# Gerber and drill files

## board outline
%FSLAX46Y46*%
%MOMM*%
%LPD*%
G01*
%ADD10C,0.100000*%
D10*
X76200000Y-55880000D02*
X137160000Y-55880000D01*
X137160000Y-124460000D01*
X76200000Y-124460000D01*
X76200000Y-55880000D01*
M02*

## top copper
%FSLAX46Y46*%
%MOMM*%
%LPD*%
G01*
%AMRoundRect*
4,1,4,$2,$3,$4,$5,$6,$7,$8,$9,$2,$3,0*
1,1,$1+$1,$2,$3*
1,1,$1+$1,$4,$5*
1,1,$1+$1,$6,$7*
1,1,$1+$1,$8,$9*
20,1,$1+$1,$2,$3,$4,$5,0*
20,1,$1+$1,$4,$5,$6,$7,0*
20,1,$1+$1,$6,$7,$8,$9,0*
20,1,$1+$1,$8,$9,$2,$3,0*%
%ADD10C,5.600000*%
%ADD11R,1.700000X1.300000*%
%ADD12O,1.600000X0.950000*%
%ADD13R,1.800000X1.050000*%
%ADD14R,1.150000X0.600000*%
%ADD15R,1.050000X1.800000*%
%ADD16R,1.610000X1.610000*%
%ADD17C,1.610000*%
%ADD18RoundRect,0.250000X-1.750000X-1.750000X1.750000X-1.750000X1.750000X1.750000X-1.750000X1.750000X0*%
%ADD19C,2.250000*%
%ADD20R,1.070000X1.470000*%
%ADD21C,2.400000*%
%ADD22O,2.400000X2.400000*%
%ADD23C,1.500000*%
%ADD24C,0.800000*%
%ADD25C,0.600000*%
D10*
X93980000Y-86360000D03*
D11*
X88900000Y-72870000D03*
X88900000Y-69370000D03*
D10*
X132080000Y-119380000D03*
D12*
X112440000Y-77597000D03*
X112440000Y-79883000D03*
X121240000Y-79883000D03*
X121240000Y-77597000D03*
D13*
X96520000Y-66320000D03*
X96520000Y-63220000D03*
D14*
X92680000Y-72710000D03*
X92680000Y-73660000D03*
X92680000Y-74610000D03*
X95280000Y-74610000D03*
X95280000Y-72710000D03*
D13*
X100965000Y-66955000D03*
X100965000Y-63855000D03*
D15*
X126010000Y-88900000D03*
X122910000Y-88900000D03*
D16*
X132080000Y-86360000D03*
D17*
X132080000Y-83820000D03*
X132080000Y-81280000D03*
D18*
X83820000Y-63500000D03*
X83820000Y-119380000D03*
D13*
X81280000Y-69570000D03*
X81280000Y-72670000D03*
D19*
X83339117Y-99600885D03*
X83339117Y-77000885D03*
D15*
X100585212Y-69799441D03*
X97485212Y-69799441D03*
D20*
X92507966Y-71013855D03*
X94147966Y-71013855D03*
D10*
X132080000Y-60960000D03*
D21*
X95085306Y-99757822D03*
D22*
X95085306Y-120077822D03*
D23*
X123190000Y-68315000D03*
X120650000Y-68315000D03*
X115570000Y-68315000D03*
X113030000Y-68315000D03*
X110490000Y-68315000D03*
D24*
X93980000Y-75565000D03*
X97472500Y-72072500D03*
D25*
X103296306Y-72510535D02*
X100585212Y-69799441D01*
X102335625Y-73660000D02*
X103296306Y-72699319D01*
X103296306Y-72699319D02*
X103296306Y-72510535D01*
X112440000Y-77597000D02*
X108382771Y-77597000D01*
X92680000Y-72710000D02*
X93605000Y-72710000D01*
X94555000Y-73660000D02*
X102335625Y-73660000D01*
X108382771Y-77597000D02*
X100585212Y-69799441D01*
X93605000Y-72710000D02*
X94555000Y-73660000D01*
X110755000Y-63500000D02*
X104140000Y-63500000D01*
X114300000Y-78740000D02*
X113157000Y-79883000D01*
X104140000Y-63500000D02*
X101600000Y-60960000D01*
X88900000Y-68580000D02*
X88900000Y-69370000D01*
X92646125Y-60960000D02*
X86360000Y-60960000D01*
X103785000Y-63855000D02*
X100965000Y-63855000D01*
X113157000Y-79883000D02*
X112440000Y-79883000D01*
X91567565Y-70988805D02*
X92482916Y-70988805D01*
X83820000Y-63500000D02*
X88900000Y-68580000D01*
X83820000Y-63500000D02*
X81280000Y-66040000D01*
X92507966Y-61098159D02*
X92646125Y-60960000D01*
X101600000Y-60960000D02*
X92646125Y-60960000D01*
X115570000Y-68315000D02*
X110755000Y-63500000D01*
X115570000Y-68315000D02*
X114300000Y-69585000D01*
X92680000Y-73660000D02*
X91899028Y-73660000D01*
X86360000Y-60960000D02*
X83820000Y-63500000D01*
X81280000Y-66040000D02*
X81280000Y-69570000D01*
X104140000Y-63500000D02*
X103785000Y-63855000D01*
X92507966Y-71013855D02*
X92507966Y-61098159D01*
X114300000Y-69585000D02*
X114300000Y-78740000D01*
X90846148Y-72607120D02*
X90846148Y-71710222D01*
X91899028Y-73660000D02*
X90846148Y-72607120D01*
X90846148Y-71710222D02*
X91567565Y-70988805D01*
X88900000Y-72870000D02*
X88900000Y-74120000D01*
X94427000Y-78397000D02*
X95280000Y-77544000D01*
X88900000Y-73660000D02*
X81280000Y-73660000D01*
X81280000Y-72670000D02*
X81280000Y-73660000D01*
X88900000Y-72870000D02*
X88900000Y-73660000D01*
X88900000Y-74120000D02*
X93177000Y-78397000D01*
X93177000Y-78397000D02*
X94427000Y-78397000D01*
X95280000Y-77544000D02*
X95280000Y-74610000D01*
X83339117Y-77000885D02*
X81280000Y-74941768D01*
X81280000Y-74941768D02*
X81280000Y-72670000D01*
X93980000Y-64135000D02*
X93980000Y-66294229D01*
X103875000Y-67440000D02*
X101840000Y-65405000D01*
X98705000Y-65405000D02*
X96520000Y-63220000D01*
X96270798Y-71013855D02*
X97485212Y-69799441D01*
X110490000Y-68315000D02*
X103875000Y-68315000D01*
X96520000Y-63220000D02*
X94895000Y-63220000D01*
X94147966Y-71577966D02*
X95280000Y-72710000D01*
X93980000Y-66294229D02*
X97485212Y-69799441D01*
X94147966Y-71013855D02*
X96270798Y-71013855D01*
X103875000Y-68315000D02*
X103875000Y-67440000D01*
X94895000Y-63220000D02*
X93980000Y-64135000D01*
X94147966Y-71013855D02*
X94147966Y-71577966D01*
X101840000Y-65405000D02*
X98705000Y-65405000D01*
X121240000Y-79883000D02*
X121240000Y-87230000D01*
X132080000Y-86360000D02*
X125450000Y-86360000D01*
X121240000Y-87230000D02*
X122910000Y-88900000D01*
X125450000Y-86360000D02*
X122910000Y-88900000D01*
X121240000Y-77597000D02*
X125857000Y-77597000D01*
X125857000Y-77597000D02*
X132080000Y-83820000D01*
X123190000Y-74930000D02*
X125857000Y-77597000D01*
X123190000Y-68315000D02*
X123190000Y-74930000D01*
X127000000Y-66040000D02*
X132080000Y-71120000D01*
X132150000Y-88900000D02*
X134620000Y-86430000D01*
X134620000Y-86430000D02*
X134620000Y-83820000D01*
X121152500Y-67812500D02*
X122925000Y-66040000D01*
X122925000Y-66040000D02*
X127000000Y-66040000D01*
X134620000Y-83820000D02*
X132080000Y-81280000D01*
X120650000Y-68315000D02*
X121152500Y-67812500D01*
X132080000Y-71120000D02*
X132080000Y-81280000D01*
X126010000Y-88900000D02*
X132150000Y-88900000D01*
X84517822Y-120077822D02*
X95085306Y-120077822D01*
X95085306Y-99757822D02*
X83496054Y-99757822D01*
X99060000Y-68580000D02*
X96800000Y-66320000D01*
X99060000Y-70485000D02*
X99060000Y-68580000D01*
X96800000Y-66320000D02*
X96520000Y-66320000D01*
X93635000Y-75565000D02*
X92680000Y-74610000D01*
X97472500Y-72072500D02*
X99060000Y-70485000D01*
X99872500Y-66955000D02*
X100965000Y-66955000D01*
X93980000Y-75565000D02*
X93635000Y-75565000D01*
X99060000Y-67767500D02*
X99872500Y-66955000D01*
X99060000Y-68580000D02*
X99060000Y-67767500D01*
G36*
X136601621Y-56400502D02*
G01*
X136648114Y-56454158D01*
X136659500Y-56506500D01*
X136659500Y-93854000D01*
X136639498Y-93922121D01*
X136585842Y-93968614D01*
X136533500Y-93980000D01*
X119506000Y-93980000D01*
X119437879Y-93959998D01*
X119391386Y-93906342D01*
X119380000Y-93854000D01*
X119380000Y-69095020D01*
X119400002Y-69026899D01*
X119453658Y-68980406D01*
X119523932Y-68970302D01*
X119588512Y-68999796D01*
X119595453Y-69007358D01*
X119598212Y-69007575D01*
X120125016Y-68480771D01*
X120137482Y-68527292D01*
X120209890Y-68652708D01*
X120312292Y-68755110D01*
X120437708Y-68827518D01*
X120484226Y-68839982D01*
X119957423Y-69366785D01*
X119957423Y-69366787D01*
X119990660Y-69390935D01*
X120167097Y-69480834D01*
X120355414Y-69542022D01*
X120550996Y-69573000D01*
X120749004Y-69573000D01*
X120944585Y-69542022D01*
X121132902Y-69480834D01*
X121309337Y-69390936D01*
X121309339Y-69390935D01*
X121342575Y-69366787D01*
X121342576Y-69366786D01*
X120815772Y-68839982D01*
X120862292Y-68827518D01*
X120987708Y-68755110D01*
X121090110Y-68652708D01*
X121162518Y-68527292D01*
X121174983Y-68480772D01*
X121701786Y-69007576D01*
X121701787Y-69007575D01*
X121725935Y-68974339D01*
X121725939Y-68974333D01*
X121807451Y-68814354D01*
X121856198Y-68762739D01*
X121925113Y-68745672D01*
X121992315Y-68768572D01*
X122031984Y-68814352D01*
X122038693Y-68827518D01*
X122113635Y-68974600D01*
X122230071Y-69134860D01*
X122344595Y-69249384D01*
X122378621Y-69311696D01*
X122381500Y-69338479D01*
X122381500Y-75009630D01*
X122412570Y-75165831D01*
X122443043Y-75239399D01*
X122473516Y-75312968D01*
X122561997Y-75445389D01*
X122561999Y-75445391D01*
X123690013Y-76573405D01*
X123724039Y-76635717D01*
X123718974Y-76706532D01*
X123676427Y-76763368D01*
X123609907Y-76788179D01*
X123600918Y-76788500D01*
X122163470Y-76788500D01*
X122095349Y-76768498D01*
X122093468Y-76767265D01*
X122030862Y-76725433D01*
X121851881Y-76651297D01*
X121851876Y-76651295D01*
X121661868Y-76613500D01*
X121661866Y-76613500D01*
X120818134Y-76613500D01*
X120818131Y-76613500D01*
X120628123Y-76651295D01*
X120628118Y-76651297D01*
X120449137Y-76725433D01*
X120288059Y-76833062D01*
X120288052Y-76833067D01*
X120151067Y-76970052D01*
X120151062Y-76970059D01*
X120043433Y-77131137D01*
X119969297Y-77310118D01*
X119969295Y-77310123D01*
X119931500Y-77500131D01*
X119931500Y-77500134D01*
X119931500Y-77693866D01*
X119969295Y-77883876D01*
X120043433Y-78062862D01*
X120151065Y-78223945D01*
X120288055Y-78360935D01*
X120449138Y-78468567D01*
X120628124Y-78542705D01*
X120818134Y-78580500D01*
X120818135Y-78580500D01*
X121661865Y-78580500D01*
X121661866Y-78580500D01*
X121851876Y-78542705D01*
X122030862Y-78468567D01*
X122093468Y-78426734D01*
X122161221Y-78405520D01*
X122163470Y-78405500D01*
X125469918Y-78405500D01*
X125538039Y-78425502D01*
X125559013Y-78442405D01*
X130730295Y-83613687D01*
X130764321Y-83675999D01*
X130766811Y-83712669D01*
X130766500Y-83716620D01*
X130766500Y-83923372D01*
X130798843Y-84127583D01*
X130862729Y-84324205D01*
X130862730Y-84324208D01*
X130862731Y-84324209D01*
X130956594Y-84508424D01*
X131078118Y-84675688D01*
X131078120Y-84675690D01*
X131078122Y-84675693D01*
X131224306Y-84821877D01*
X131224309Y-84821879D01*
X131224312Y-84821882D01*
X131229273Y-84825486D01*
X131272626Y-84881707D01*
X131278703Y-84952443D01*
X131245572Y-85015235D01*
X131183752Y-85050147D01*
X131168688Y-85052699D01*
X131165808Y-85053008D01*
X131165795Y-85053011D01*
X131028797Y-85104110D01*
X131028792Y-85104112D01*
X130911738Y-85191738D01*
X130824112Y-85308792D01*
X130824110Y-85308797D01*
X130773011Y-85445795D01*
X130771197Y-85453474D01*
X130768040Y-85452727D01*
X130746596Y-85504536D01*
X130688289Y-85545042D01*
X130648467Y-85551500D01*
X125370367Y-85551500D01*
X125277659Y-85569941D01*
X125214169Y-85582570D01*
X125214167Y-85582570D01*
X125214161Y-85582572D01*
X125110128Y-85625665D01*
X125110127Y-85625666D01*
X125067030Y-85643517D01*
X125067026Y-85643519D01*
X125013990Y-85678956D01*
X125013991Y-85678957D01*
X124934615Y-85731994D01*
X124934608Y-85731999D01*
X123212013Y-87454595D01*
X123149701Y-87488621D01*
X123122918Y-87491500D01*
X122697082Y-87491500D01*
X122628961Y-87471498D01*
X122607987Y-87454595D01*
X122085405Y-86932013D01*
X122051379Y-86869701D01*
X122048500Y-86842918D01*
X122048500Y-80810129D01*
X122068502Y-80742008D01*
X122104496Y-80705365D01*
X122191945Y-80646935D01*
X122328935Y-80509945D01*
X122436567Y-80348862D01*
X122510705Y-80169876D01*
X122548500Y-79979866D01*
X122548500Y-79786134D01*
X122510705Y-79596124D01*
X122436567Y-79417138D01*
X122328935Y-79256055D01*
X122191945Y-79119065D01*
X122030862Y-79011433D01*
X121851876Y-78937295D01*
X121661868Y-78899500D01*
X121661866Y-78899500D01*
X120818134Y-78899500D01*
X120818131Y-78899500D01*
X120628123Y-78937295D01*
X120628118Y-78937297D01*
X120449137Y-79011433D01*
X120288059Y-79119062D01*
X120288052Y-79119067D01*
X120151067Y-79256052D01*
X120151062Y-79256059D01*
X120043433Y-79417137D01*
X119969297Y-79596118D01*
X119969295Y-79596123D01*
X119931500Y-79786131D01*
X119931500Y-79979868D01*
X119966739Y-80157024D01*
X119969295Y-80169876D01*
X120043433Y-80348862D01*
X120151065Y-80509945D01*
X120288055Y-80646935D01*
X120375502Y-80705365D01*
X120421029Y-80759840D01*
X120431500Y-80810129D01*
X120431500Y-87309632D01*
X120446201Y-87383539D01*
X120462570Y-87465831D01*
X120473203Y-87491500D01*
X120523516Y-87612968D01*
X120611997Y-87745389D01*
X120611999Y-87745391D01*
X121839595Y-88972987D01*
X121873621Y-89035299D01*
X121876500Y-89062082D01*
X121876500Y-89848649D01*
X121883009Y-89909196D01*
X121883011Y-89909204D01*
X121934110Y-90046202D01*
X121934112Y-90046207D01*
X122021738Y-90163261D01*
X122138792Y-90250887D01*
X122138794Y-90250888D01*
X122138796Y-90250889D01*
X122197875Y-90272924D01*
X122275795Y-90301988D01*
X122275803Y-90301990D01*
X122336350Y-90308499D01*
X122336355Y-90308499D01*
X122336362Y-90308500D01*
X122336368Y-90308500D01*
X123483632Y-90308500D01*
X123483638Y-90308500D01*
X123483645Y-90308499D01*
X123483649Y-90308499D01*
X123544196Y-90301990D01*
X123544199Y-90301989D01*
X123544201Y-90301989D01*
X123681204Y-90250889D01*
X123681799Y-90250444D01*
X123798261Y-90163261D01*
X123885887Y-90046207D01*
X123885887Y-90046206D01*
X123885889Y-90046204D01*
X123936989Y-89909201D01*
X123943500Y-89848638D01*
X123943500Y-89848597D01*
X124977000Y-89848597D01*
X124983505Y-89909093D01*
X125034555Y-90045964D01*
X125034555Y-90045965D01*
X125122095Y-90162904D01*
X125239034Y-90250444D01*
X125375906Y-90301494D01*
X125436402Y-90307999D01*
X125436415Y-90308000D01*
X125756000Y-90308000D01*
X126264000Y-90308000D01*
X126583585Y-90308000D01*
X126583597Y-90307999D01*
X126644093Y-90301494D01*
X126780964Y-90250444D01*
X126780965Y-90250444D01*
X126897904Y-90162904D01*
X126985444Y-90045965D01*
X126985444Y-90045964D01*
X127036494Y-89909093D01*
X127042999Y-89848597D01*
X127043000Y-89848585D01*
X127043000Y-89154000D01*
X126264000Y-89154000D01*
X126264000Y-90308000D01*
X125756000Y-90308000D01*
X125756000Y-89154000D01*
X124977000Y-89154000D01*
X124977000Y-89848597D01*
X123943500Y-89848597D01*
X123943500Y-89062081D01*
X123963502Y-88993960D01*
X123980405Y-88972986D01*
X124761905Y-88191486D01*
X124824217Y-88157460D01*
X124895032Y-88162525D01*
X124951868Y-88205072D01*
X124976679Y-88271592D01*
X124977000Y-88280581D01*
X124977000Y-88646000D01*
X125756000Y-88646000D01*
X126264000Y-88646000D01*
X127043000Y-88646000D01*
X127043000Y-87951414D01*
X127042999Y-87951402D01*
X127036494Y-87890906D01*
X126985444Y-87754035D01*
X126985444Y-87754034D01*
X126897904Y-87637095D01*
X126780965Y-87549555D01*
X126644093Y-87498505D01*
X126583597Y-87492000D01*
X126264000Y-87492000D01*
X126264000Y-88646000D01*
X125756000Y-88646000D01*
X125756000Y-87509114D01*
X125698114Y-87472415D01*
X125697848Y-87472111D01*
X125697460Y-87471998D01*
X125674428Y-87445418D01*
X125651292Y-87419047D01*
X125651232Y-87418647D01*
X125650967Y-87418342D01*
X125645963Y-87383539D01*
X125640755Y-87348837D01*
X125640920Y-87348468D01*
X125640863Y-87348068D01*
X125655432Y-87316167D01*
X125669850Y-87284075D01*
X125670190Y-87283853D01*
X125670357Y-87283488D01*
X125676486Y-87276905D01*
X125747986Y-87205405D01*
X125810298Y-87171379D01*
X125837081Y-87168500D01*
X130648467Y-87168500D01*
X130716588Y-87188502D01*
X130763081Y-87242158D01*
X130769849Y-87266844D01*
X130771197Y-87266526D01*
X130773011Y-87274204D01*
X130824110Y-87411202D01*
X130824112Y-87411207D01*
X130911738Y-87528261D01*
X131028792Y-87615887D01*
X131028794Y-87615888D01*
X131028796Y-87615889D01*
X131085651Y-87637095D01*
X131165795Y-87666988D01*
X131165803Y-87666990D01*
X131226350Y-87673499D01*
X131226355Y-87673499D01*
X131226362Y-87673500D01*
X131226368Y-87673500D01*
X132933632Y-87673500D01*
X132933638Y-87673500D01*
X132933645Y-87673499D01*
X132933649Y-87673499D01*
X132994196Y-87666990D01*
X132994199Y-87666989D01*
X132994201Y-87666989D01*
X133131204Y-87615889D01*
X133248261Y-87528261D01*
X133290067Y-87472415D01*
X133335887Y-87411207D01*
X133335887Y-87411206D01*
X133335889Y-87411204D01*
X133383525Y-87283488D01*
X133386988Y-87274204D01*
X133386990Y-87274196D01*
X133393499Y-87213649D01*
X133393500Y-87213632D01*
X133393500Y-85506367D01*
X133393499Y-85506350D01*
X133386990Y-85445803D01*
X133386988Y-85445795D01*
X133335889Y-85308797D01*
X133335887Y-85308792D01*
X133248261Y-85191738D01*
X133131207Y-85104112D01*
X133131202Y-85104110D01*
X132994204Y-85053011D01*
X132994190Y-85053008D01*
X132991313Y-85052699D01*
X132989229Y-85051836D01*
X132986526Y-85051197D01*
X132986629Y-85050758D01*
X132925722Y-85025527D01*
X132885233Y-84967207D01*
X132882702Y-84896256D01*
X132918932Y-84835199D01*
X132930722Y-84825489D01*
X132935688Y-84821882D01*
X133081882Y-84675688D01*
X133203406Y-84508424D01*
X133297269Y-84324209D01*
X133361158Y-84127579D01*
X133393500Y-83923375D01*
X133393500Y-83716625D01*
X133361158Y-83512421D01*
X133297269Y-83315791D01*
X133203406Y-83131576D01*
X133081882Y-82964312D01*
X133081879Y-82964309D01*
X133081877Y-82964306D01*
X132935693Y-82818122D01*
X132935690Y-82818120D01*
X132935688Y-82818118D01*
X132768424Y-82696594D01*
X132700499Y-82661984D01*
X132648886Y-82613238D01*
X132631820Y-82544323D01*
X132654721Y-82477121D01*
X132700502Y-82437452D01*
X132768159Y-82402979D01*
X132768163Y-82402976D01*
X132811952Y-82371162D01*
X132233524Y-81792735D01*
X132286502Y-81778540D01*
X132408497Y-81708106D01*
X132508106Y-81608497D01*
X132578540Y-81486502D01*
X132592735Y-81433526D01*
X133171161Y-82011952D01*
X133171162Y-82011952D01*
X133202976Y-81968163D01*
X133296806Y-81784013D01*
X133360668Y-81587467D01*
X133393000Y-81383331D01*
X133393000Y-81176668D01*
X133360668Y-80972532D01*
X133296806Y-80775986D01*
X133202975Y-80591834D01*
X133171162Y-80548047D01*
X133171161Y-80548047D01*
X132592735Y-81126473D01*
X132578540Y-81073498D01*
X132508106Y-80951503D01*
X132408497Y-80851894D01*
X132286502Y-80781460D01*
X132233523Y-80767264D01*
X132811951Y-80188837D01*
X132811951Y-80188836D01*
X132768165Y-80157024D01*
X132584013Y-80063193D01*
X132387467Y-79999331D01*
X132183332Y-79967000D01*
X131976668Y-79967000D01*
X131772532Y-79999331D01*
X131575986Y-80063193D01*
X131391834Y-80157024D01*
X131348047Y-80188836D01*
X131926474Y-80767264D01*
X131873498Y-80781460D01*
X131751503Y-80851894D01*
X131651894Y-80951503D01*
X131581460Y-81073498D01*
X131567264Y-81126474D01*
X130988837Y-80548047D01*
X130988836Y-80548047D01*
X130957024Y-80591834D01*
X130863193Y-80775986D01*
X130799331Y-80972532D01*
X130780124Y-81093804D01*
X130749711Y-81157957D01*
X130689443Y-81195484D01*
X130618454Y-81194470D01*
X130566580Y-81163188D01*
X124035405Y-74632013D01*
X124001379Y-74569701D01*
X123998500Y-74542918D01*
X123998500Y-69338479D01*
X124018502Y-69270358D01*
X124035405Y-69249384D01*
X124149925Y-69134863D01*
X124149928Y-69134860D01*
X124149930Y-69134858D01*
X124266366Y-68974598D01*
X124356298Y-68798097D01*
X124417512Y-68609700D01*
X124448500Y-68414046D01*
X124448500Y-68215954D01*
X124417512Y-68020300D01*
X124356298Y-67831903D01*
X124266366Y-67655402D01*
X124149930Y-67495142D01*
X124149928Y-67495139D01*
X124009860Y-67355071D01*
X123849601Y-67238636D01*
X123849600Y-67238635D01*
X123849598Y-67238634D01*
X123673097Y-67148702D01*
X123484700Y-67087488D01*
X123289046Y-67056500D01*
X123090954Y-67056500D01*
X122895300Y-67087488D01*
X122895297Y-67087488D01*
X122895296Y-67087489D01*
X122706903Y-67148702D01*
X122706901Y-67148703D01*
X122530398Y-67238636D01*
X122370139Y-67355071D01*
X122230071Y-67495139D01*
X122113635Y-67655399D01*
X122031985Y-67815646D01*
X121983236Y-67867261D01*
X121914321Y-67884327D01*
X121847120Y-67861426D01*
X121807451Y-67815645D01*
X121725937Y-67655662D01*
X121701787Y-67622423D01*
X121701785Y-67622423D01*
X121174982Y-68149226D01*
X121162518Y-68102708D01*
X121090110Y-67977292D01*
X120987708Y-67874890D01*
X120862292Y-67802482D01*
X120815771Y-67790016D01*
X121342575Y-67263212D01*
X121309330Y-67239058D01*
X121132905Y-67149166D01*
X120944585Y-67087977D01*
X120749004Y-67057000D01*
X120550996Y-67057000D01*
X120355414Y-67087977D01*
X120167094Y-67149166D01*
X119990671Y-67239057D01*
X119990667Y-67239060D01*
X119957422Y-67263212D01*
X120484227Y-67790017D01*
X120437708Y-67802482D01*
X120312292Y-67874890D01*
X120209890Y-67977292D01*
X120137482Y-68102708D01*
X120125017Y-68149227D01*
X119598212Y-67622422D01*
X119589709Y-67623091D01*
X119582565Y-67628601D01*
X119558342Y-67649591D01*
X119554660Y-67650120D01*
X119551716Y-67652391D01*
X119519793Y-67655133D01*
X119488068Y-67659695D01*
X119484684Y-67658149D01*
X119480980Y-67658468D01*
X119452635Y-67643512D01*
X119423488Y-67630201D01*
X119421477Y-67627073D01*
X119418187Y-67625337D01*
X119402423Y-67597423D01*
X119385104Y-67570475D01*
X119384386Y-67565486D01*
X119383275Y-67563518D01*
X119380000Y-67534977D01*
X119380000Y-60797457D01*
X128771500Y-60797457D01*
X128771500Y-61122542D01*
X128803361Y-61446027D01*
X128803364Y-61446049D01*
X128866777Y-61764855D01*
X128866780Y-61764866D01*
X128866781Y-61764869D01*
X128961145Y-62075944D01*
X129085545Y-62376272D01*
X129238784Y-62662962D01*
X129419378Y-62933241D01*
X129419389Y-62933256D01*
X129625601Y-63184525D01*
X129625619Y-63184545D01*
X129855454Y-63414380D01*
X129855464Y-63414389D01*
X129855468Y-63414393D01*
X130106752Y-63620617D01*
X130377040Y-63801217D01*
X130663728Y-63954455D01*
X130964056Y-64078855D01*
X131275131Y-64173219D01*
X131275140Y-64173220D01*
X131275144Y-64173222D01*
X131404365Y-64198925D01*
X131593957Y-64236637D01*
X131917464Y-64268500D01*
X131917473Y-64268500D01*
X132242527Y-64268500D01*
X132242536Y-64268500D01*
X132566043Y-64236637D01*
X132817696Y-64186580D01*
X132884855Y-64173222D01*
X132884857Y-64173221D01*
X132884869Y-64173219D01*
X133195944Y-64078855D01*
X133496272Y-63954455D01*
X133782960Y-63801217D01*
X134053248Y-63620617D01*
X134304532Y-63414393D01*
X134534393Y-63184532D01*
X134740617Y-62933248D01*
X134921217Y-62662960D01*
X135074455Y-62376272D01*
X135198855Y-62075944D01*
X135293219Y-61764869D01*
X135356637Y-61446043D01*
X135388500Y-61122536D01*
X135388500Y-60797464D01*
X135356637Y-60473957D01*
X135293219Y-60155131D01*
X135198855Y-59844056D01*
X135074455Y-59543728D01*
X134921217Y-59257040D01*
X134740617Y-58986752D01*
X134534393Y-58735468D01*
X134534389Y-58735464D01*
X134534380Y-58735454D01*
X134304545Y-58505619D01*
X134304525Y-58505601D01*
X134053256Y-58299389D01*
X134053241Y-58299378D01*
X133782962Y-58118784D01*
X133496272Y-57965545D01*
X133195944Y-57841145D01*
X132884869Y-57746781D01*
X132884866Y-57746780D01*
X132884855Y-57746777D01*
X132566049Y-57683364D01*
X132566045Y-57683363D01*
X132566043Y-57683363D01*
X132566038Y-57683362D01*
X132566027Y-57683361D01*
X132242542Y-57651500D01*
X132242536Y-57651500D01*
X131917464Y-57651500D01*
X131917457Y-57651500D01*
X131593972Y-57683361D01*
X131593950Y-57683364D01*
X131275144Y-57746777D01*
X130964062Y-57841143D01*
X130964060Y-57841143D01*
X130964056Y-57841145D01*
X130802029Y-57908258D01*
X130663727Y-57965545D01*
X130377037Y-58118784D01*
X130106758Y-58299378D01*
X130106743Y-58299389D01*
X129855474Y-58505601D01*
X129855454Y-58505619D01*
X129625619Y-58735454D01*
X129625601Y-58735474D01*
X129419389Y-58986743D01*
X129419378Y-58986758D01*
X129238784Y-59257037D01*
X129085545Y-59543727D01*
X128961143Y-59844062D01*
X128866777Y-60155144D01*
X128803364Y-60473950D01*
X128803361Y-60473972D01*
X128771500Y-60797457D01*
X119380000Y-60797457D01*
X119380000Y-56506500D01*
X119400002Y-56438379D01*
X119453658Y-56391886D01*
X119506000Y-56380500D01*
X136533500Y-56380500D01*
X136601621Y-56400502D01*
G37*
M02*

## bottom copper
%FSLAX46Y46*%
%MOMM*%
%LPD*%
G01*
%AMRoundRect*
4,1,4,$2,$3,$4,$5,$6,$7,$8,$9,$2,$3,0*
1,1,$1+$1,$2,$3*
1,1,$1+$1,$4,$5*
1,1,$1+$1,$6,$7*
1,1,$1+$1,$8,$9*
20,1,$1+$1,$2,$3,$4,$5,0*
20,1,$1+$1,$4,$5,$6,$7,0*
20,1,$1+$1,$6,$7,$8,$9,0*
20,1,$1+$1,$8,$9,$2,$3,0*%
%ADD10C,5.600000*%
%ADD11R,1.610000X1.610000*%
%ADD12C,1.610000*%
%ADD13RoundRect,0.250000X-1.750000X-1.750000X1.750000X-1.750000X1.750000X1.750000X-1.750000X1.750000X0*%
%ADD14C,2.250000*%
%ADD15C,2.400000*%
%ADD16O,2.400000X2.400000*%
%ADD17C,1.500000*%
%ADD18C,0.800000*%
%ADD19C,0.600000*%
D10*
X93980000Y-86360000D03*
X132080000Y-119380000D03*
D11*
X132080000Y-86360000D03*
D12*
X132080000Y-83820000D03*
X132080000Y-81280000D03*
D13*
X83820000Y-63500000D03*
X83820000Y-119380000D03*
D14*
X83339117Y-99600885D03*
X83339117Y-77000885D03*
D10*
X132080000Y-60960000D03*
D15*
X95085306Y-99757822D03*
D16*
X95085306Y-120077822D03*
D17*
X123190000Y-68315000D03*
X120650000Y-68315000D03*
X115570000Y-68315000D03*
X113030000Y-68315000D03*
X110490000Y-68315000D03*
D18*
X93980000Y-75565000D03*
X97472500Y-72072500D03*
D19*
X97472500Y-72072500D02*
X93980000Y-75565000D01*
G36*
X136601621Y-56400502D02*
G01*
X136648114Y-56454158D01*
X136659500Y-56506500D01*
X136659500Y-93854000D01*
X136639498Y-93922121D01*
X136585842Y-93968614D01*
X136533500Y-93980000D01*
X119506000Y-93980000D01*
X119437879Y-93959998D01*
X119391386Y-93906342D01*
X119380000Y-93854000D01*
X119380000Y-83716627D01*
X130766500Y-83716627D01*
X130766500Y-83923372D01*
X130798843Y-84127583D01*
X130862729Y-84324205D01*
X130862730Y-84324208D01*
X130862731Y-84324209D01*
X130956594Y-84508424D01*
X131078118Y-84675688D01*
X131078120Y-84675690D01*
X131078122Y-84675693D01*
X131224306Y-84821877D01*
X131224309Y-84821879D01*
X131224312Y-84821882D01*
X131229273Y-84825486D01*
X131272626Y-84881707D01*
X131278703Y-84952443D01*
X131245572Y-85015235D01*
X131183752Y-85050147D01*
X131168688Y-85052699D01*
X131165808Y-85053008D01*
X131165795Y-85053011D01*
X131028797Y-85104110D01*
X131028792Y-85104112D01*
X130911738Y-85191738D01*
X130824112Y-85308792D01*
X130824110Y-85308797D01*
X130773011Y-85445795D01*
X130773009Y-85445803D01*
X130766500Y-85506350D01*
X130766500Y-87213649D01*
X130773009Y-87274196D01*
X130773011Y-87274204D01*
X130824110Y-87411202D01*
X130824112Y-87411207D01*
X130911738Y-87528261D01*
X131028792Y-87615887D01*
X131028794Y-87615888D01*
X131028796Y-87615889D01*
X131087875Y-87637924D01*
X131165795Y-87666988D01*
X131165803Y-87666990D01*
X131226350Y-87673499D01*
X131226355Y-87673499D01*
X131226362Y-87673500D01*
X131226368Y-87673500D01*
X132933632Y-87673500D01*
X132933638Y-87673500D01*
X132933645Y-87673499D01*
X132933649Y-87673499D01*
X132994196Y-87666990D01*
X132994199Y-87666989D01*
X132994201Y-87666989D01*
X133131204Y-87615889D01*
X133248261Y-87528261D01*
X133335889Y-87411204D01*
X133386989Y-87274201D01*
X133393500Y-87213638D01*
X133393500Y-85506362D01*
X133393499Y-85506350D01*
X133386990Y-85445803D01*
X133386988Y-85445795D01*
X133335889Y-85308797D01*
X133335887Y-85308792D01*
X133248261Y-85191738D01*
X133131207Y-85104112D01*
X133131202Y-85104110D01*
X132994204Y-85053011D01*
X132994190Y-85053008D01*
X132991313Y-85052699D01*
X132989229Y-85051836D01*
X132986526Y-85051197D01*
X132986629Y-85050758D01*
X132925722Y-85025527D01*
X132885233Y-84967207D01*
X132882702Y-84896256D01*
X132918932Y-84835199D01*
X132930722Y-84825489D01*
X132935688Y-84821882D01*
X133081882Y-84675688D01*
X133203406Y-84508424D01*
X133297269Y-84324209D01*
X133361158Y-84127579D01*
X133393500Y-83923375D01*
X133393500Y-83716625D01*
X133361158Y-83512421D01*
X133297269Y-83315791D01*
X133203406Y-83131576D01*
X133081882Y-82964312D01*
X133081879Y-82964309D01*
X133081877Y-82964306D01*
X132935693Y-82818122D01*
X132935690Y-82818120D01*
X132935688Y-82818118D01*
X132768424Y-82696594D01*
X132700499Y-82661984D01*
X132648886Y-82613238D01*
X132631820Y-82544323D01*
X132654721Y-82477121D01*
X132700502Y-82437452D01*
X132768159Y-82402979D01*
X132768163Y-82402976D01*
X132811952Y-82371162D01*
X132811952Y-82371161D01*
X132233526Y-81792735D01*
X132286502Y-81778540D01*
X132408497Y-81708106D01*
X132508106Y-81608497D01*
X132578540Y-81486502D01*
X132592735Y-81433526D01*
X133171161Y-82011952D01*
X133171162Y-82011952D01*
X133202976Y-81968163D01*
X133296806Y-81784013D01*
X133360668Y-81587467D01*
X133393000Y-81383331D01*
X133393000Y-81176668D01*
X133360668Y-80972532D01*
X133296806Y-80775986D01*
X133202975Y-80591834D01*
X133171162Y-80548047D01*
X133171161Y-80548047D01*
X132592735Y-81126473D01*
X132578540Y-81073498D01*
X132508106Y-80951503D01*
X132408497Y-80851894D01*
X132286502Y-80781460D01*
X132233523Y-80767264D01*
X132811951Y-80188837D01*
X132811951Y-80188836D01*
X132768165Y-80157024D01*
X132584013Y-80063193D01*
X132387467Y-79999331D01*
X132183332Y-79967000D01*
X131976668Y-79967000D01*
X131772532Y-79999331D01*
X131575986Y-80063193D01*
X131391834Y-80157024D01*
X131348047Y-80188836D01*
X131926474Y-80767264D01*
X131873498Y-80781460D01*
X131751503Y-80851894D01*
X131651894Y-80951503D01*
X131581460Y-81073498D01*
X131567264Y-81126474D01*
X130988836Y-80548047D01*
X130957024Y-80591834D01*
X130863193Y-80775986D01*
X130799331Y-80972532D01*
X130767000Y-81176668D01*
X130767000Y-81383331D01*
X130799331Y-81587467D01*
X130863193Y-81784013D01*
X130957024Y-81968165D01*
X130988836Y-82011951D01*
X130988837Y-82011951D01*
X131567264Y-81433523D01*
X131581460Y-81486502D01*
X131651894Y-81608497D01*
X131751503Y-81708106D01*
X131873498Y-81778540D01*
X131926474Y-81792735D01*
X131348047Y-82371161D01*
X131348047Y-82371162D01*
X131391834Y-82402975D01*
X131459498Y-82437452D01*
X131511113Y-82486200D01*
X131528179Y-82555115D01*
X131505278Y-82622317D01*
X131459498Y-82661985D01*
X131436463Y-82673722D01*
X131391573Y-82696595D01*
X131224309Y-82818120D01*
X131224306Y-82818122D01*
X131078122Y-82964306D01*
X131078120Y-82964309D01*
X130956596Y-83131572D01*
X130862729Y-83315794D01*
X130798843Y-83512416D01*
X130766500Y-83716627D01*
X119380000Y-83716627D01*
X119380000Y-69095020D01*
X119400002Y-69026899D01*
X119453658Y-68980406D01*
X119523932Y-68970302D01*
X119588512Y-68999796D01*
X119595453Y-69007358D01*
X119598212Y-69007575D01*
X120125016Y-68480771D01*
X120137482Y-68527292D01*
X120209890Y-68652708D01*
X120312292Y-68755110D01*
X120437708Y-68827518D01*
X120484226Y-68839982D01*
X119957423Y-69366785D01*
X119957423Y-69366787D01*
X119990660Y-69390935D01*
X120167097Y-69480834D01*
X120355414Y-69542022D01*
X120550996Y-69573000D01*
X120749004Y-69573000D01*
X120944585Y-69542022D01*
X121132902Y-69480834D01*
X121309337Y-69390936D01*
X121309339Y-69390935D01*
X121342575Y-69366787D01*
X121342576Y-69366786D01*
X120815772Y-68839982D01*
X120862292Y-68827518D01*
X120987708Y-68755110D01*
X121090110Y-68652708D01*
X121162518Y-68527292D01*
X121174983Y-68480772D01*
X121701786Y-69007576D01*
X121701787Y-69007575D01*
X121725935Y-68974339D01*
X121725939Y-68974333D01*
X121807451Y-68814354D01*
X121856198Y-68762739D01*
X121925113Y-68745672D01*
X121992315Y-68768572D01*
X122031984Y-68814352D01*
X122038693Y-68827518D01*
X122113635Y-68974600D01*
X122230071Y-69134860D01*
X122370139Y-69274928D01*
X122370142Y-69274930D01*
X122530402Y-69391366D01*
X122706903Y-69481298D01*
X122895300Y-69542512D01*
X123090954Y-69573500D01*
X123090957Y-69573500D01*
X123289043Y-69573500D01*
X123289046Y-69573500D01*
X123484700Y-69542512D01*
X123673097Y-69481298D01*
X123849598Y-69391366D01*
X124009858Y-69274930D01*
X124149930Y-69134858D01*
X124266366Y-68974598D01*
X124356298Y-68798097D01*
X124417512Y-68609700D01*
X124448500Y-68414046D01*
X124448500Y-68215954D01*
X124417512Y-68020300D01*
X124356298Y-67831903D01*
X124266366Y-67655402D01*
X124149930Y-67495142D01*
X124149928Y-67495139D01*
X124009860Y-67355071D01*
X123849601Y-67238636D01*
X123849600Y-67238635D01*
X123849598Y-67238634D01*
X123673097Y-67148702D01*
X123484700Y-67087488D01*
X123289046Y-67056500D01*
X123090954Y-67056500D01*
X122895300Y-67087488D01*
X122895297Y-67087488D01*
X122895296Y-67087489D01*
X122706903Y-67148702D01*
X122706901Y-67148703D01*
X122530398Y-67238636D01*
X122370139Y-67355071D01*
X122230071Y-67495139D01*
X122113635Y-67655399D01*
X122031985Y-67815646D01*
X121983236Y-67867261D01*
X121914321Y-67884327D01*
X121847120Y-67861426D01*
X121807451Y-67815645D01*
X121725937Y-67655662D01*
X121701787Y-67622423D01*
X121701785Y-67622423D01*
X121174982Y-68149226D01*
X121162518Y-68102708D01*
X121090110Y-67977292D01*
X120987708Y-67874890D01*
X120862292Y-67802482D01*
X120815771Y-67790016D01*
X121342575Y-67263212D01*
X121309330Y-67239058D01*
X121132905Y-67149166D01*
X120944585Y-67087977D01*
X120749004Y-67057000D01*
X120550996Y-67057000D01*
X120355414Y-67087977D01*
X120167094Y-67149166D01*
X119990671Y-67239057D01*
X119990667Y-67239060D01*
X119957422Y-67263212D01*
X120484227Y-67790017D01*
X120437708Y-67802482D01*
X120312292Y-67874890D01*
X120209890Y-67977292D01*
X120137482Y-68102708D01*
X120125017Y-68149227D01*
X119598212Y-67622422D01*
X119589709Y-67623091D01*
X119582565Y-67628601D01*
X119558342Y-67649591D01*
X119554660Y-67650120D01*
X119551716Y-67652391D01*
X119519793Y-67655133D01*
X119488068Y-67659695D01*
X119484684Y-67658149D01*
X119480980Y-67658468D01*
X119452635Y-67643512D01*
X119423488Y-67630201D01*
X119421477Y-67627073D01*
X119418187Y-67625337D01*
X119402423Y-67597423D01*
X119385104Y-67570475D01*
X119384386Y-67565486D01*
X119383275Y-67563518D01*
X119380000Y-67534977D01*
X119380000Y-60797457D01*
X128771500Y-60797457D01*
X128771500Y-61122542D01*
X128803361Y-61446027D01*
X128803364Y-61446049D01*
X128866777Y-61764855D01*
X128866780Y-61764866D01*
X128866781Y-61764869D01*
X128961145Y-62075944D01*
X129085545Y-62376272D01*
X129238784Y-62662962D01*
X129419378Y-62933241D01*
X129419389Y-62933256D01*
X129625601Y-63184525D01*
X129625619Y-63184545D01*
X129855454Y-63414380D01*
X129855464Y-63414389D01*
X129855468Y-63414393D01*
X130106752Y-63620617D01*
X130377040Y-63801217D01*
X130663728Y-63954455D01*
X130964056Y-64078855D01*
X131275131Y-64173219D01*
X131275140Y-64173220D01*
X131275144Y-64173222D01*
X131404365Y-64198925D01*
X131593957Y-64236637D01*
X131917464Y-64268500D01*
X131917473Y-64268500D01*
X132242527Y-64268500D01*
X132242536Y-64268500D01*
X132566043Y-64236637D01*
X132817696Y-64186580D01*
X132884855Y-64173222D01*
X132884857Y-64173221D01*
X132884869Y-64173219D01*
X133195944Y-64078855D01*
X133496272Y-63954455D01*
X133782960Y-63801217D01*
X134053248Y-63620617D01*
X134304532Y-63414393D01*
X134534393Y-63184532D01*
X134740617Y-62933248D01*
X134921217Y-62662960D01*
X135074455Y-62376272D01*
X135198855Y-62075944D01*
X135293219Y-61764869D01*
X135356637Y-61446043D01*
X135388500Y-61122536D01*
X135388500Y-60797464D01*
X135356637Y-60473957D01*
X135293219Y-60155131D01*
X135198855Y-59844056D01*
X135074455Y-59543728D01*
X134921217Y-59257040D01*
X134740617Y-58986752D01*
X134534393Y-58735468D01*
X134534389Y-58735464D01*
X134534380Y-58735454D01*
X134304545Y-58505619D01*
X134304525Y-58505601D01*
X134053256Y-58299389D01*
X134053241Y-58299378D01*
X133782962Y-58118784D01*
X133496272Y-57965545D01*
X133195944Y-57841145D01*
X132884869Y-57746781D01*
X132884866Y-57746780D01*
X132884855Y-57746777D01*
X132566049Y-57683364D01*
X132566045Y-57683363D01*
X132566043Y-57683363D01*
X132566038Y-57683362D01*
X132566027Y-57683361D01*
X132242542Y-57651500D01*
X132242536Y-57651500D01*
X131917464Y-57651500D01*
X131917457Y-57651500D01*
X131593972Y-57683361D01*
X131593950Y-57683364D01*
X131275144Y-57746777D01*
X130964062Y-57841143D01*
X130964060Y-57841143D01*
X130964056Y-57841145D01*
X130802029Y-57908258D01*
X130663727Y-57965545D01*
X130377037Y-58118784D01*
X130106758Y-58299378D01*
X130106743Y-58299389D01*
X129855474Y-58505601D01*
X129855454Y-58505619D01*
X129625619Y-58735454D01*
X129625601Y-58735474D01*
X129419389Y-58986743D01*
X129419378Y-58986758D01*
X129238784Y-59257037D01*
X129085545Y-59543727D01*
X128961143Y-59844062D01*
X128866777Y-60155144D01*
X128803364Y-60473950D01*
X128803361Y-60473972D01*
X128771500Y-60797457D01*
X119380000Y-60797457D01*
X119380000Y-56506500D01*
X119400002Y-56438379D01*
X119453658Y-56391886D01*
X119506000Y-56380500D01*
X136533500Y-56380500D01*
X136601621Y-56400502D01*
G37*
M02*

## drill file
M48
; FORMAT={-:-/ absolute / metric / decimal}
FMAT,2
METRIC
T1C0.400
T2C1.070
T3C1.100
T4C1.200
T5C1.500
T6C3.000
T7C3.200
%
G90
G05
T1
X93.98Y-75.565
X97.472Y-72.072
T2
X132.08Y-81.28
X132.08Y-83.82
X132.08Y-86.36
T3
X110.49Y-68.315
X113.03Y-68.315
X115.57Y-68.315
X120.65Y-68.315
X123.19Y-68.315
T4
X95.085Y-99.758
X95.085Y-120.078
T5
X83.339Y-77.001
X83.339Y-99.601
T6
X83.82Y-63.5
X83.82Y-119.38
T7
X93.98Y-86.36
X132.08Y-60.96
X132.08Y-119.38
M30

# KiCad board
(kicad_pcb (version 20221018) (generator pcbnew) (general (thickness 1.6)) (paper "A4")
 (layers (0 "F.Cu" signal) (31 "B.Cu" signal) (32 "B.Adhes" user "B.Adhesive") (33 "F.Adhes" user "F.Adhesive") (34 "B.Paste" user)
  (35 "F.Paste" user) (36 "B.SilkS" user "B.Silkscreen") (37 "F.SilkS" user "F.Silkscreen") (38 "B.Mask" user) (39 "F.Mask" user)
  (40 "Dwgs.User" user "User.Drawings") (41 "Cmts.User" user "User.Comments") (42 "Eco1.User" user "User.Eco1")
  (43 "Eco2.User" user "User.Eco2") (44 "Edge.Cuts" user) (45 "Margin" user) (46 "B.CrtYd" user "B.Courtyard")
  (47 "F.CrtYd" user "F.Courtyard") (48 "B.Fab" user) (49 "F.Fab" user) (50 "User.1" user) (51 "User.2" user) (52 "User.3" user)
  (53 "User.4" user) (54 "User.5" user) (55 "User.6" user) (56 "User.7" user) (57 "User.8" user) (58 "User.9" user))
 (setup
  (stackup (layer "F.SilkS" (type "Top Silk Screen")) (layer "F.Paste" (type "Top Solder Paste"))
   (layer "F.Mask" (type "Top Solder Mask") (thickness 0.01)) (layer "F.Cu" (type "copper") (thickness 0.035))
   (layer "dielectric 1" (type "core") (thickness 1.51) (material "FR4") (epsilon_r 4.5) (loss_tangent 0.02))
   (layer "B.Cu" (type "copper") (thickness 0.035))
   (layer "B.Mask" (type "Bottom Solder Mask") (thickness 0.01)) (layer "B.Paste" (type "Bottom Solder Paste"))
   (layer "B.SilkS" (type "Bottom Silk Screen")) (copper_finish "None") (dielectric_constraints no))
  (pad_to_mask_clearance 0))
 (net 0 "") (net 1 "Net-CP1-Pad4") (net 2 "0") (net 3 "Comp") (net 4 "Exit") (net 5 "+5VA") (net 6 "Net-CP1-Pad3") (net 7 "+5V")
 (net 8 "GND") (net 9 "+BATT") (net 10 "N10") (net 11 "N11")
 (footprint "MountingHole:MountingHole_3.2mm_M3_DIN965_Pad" (layer "F.Cu") (at 93.98 86.36)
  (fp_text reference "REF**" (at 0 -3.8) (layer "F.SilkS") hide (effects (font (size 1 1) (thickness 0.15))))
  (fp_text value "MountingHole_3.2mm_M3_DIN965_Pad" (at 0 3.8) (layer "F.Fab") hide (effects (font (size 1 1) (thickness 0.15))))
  (pad "1" thru_hole circle (at 0 0) (size 5.6 5.6) (drill 3.2) (layers "*.Cu" "*.Mask")))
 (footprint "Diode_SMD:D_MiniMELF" (layer "F.Cu") (at 88.9 71.12 90)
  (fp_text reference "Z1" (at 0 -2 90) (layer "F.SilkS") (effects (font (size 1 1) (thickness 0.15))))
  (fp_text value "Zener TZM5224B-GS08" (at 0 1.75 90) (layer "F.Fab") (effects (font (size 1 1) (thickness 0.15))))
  (pad "1" smd rect (at -1.75 0 90) (size 1.3 1.7) (layers "F.Cu" "F.Paste" "F.Mask") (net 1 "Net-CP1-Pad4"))
  (pad "2" smd rect (at 1.75 0 90) (size 1.3 1.7) (layers "F.Cu" "F.Paste" "F.Mask") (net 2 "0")))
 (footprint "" (layer "F.Cu") (at 132.08 119.38)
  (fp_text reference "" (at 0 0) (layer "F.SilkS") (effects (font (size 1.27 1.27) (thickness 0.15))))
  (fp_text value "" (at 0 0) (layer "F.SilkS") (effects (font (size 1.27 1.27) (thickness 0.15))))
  (pad "1" thru_hole circle (at 0 0) (size 5.6 5.6) (drill 3.2) (layers "*.Cu" "*.Mask")))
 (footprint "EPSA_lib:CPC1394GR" (layer "F.Cu") (at 116.84 78.74 -90)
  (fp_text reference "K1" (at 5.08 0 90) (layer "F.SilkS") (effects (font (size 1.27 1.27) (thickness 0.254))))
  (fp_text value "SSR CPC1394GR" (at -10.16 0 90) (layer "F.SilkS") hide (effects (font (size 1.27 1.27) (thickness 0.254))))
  (pad "1" smd oval (at -1.143 4.4 270) (size 0.95 1.6) (layers "F.Cu" "F.Paste" "F.Mask") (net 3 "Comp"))
  (pad "2" smd oval (at 1.143 4.4 270) (size 0.95 1.6) (layers "F.Cu" "F.Paste" "F.Mask") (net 2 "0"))
  (pad "3" smd oval (at 1.143 -4.4 270) (size 0.95 1.6) (layers "F.Cu" "F.Paste" "F.Mask") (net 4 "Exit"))
  (pad "4" smd oval (at -1.143 -4.4 270) (size 0.95 1.6) (layers "F.Cu" "F.Paste" "F.Mask") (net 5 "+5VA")))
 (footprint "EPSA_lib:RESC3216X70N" (layer "F.Cu") (at 96.52 64.77 90)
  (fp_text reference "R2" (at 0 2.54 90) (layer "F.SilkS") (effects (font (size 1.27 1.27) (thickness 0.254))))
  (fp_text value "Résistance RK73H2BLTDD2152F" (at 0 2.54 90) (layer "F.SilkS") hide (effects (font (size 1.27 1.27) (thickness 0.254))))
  (pad "1" smd rect (at -1.55 0 90) (size 1.05 1.8) (layers "F.Cu" "F.Paste" "F.Mask") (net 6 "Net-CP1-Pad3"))
  (pad "2" smd rect (at 1.55 0 90) (size 1.05 1.8) (layers "F.Cu" "F.Paste" "F.Mask") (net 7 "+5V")))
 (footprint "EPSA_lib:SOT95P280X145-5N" (layer "F.Cu") (at 93.98 73.66)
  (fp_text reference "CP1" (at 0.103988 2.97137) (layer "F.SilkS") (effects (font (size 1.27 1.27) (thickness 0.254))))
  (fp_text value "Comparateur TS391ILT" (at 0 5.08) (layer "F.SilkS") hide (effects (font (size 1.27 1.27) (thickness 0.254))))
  (pad "1" smd rect (at -1.3 -0.95 90) (size 0.6 1.15) (layers "F.Cu" "F.Paste" "F.Mask") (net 3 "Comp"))
  (pad "2" smd rect (at -1.3 0 90) (size 0.6 1.15) (layers "F.Cu" "F.Paste" "F.Mask") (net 2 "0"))
  (pad "3" smd rect (at -1.3 0.95 90) (size 0.6 1.15) (layers "F.Cu" "F.Paste" "F.Mask") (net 6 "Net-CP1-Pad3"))
  (pad "4" smd rect (at 1.3 0.95 90) (size 0.6 1.15) (layers "F.Cu" "F.Paste" "F.Mask") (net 1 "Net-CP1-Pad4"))
  (pad "5" smd rect (at 1.3 -0.95 90) (size 0.6 1.15) (layers "F.Cu" "F.Paste" "F.Mask") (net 7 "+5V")))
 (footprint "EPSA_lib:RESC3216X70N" (layer "F.Cu") (at 100.965 65.405 90)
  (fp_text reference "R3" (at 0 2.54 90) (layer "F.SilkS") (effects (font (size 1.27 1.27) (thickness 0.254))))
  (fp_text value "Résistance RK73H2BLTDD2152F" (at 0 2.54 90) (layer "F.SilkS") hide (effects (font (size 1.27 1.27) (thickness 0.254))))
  (pad "1" smd rect (at -1.55 0 90) (size 1.05 1.8) (layers "F.Cu" "F.Paste" "F.Mask") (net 6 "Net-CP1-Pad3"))
  (pad "2" smd rect (at 1.55 0 90) (size 1.05 1.8) (layers "F.Cu" "F.Paste" "F.Mask") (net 2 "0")))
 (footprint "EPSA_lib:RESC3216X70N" (layer "F.Cu") (at 124.46 88.9 180)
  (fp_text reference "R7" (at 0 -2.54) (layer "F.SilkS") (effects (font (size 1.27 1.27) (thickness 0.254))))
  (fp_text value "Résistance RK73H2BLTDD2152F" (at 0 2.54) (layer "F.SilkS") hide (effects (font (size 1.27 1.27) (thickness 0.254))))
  (pad "1" smd rect (at -1.55 0 180) (size 1.05 1.8) (layers "F.Cu" "F.Paste" "F.Mask") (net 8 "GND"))
  (pad "2" smd rect (at 1.55 0 180) (size 1.05 1.8) (layers "F.Cu" "F.Paste" "F.Mask") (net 4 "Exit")))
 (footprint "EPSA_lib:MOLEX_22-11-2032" (layer "F.Cu") (at 132.08 86.36 90)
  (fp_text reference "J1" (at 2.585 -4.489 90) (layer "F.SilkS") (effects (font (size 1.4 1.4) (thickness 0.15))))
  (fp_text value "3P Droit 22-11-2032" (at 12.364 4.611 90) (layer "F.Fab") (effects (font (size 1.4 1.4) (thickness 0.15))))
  (pad "1" thru_hole rect (at 0 0 90) (size 1.61 1.61) (drill 1.07) (layers "*.Cu" "*.Mask") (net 4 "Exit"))
  (pad "2" thru_hole circle (at 2.54 0 90) (size 1.61 1.61) (drill 1.07) (layers "*.Cu" "*.Mask") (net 5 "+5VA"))
  (pad "3" thru_hole circle (at 5.08 0 90) (size 1.61 1.61) (drill 1.07) (layers "*.Cu" "*.Mask") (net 8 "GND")))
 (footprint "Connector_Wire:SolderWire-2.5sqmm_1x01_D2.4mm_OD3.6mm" (layer "F.Cu") (at 83.82 63.5)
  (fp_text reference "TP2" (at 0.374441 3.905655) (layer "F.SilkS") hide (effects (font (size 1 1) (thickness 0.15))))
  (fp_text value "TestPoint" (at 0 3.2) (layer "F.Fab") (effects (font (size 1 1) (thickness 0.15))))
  (pad "1" thru_hole roundrect (at 0 0) (size 4 4) (drill 3) (layers "*.Cu" "*.Mask") (roundrect_rratio 0.0625) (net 2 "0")))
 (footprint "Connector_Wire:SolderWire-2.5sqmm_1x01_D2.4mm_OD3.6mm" (layer "F.Cu") (at 83.82 119.38)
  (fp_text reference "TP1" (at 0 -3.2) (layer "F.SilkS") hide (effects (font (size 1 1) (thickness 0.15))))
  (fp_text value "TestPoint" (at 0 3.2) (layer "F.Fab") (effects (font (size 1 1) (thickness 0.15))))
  (pad "1" thru_hole roundrect (at 0 0) (size 4 4) (drill 3) (layers "*.Cu" "*.Mask") (roundrect_rratio 0.0625) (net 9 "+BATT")))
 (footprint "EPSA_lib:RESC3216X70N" (layer "F.Cu") (at 81.28 71.12 -90)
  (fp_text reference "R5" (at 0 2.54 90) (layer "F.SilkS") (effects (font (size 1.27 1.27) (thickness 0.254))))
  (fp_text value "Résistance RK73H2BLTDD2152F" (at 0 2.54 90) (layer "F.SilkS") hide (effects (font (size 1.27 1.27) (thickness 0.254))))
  (pad "1" smd rect (at -1.55 0 270) (size 1.05 1.8) (layers "F.Cu" "F.Paste" "F.Mask") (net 2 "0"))
  (pad "2" smd rect (at 1.55 0 270) (size 1.05 1.8) (layers "F.Cu" "F.Paste" "F.Mask") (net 1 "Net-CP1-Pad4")))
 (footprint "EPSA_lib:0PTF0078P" (layer "F.Cu") (at 83.339117 88.300885 90)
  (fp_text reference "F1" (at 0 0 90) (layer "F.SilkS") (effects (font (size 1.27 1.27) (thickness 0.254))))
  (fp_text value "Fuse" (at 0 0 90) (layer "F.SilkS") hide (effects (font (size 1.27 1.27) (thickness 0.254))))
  (pad "1" thru_hole circle (at -11.3 0 90) (size 2.25 2.25) (drill 1.5) (layers "*.Cu" "*.Mask") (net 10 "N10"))
  (pad "2" thru_hole circle (at 11.3 0 90) (size 2.25 2.25) (drill 1.5) (layers "*.Cu" "*.Mask") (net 1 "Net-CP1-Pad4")))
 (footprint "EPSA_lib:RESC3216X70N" (layer "F.Cu") (at 99.035212 69.799441 180)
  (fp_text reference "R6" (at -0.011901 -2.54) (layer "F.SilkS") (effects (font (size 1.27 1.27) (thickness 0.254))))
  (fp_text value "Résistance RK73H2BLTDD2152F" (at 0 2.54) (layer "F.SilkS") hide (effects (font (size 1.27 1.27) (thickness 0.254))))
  (pad "1" smd rect (at -1.55 0 180) (size 1.05 1.8) (layers "F.Cu" "F.Paste" "F.Mask") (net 3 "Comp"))
  (pad "2" smd rect (at 1.55 0 180) (size 1.05 1.8) (layers "F.Cu" "F.Paste" "F.Mask") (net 7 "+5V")))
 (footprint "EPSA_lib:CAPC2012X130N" (layer "F.Cu") (at 93.327966 71.013855)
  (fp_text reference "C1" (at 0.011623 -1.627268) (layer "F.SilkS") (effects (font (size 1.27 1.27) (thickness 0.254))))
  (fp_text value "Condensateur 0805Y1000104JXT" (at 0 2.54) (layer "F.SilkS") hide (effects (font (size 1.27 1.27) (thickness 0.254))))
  (pad "1" smd rect (at -0.82 0) (size 1.07 1.47) (layers "F.Cu" "F.Paste" "F.Mask") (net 2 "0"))
  (pad "2" smd rect (at 0.82 0) (size 1.07 1.47) (layers "F.Cu" "F.Paste" "F.Mask") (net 7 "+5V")))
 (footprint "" (layer "F.Cu") (at 132.08 60.96)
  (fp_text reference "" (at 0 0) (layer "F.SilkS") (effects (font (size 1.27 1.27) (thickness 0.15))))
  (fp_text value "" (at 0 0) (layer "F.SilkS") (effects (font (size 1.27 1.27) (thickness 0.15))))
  (pad "1" thru_hole circle (at 0 0) (size 5.6 5.6) (drill 3.2) (layers "*.Cu" "*.Mask")))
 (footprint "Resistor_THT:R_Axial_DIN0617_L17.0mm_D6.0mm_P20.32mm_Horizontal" (layer "F.Cu") (at 95.085306 99.757822 -90)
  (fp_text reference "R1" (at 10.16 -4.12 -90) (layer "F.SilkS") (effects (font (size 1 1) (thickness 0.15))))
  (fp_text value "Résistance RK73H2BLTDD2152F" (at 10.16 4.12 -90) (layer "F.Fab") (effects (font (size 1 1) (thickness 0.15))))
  (pad "1" thru_hole circle (at 0 0 270) (size 2.4 2.4) (drill 1.2) (layers "*.Cu" "*.Mask") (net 10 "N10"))
  (pad "2" thru_hole oval (at 20.32 0 270) (size 2.4 2.4) (drill 1.2) (layers "*.Cu" "*.Mask") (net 9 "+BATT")))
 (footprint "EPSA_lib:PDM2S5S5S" (layer "F.Cu") (at 123.19 68.315 180)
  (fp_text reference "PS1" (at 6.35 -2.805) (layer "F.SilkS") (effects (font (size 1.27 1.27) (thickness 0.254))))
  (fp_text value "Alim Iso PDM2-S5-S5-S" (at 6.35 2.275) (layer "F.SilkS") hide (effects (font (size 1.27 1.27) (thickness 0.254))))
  (pad "1" thru_hole circle (at 0 0 180) (size 1.5 1.5) (drill 1.1) (layers "*.Cu" "*.Mask") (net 5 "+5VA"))
  (pad "2" thru_hole circle (at 2.54 0 180) (size 1.5 1.5) (drill 1.1) (layers "*.Cu" "*.Mask") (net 8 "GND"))
  (pad "4" thru_hole circle (at 7.62 0 180) (size 1.5 1.5) (drill 1.1) (layers "*.Cu" "*.Mask") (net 2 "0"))
  (pad "5" thru_hole circle (at 10.16 0 180) (size 1.5 1.5) (drill 1.1) (layers "*.Cu" "*.Mask") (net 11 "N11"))
  (pad "6" thru_hole circle (at 12.7 0 180) (size 1.5 1.5) (drill 1.1) (layers "*.Cu" "*.Mask") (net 7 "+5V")))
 (gr_rect (start 76.2 55.88) (end 137.16 124.46) (stroke (width 0.1) (type solid)) (fill none) (layer "Edge.Cuts"))
 (segment (start 103.296306 72.510535) (end 100.585212 69.799441) (width 0.6) (layer "F.Cu") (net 3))
 (segment (start 102.335625 73.66) (end 103.296306 72.699319) (width 0.6) (layer "F.Cu") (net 3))
 (segment (start 103.296306 72.699319) (end 103.296306 72.510535) (width 0.6) (layer "F.Cu") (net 3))
 (segment (start 112.44 77.597) (end 108.382771 77.597) (width 0.6) (layer "F.Cu") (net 3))
 (segment (start 92.68 72.71) (end 93.605 72.71) (width 0.6) (layer "F.Cu") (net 3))
 (segment (start 94.555 73.66) (end 102.335625 73.66) (width 0.6) (layer "F.Cu") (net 3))
 (segment (start 108.382771 77.597) (end 100.585212 69.799441) (width 0.6) (layer "F.Cu") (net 3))
 (segment (start 93.605 72.71) (end 94.555 73.66) (width 0.6) (layer "F.Cu") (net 3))
 (segment (start 110.755 63.5) (end 104.14 63.5) (width 0.6) (layer "F.Cu") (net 2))
 (segment (start 114.3 78.74) (end 113.157 79.883) (width 0.6) (layer "F.Cu") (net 2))
 (segment (start 104.14 63.5) (end 101.6 60.96) (width 0.6) (layer "F.Cu") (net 2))
 (segment (start 88.9 68.58) (end 88.9 69.37) (width 0.6) (layer "F.Cu") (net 2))
 (segment (start 92.646125 60.96) (end 86.36 60.96) (width 0.6) (layer "F.Cu") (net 2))
 (segment (start 103.785 63.855) (end 100.965 63.855) (width 0.6) (layer "F.Cu") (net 2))
 (segment (start 113.157 79.883) (end 112.44 79.883) (width 0.6) (layer "F.Cu") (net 2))
 (segment (start 91.567565 70.988805) (end 92.482916 70.988805) (width 0.6) (layer "F.Cu") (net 2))
 (segment (start 83.82 63.5) (end 88.9 68.58) (width 0.6) (layer "F.Cu") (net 2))
 (segment (start 83.82 63.5) (end 81.28 66.04) (width 0.6) (layer "F.Cu") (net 2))
 (segment (start 92.507966 61.098159) (end 92.646125 60.96) (width 0.6) (layer "F.Cu") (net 2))
 (segment (start 101.6 60.96) (end 92.646125 60.96) (width 0.6) (layer "F.Cu") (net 2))
 (segment (start 115.57 68.315) (end 110.755 63.5) (width 0.6) (layer "F.Cu") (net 2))
 (segment (start 115.57 68.315) (end 114.3 69.585) (width 0.6) (layer "F.Cu") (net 2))
 (segment (start 92.68 73.66) (end 91.899028 73.66) (width 0.6) (layer "F.Cu") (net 2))
 (segment (start 86.36 60.96) (end 83.82 63.5) (width 0.6) (layer "F.Cu") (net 2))
 (segment (start 81.28 66.04) (end 81.28 69.57) (width 0.6) (layer "F.Cu") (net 2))
 (segment (start 104.14 63.5) (end 103.785 63.855) (width 0.6) (layer "F.Cu") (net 2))
 (segment (start 92.507966 71.013855) (end 92.507966 61.098159) (width 0.6) (layer "F.Cu") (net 2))
 (segment (start 114.3 69.585) (end 114.3 78.74) (width 0.6) (layer "F.Cu") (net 2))
 (segment (start 90.846148 72.60712) (end 90.846148 71.710222) (width 0.6) (layer "F.Cu") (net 2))
 (segment (start 91.899028 73.66) (end 90.846148 72.60712) (width 0.6) (layer "F.Cu") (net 2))
 (segment (start 90.846148 71.710222) (end 91.567565 70.988805) (width 0.6) (layer "F.Cu") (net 2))
 (segment (start 88.9 72.87) (end 88.9 74.12) (width 0.6) (layer "F.Cu") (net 1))
 (segment (start 94.427 78.397) (end 95.28 77.544) (width 0.6) (layer "F.Cu") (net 1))
 (segment (start 88.9 73.66) (end 81.28 73.66) (width 0.6) (layer "F.Cu") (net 1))
 (segment (start 81.28 72.67) (end 81.28 73.66) (width 0.6) (layer "F.Cu") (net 1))
 (segment (start 88.9 72.87) (end 88.9 73.66) (width 0.6) (layer "F.Cu") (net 1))
 (segment (start 88.9 74.12) (end 93.177 78.397) (width 0.6) (layer "F.Cu") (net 1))
 (segment (start 93.177 78.397) (end 94.427 78.397) (width 0.6) (layer "F.Cu") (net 1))
 (segment (start 95.28 77.544) (end 95.28 74.61) (width 0.6) (layer "F.Cu") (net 1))
 (segment (start 83.339117 77.000885) (end 81.28 74.941768) (width 0.6) (layer "F.Cu") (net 1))
 (segment (start 81.28 74.941768) (end 81.28 72.67) (width 0.6) (layer "F.Cu") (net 1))
 (segment (start 93.98 64.135) (end 93.98 66.294229) (width 0.6) (layer "F.Cu") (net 7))
 (segment (start 103.875 67.44) (end 101.84 65.405) (width 0.6) (layer "F.Cu") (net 7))
 (segment (start 98.705 65.405) (end 96.52 63.22) (width 0.6) (layer "F.Cu") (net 7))
 (segment (start 96.270798 71.013855) (end 97.485212 69.799441) (width 0.6) (layer "F.Cu") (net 7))
 (segment (start 110.49 68.315) (end 103.875 68.315) (width 0.6) (layer "F.Cu") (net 7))
 (segment (start 96.52 63.22) (end 94.895 63.22) (width 0.6) (layer "F.Cu") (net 7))
 (segment (start 94.147966 71.577966) (end 95.28 72.71) (width 0.6) (layer "F.Cu") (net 7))
 (segment (start 93.98 66.294229) (end 97.485212 69.799441) (width 0.6) (layer "F.Cu") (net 7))
 (segment (start 94.147966 71.013855) (end 96.270798 71.013855) (width 0.6) (layer "F.Cu") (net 7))
 (segment (start 103.875 68.315) (end 103.875 67.44) (width 0.6) (layer "F.Cu") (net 7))
 (segment (start 94.895 63.22) (end 93.98 64.135) (width 0.6) (layer "F.Cu") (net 7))
 (segment (start 94.147966 71.013855) (end 94.147966 71.577966) (width 0.6) (layer "F.Cu") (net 7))
 (segment (start 101.84 65.405) (end 98.705 65.405) (width 0.6) (layer "F.Cu") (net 7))
 (segment (start 121.24 79.883) (end 121.24 87.23) (width 0.6) (layer "F.Cu") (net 4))
 (segment (start 132.08 86.36) (end 125.45 86.36) (width 0.6) (layer "F.Cu") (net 4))
 (segment (start 121.24 87.23) (end 122.91 88.9) (width 0.6) (layer "F.Cu") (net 4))
 (segment (start 125.45 86.36) (end 122.91 88.9) (width 0.6) (layer "F.Cu") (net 4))
 (segment (start 121.24 77.597) (end 125.857 77.597) (width 0.6) (layer "F.Cu") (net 5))
 (segment (start 125.857 77.597) (end 132.08 83.82) (width 0.6) (layer "F.Cu") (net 5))
 (segment (start 123.19 74.93) (end 125.857 77.597) (width 0.6) (layer "F.Cu") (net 5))
 (segment (start 123.19 68.315) (end 123.19 74.93) (width 0.6) (layer "F.Cu") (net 5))
 (segment (start 127 66.04) (end 132.08 71.12) (width 0.6) (layer "F.Cu") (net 8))
 (segment (start 132.15 88.9) (end 134.62 86.43) (width 0.6) (layer "F.Cu") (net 8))
 (segment (start 134.62 86.43) (end 134.62 83.82) (width 0.6) (layer "F.Cu") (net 8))
 (segment (start 121.1525 67.8125) (end 122.925 66.04) (width 0.6) (layer "F.Cu") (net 8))
 (segment (start 122.925 66.04) (end 127 66.04) (width 0.6) (layer "F.Cu") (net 8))
 (segment (start 134.62 83.82) (end 132.08 81.28) (width 0.6) (layer "F.Cu") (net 8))
 (segment (start 120.65 68.315) (end 121.1525 67.8125) (width 0.6) (layer "F.Cu") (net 8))
 (segment (start 132.08 71.12) (end 132.08 81.28) (width 0.6) (layer "F.Cu") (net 8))
 (segment (start 126.01 88.9) (end 132.15 88.9) (width 0.6) (layer "F.Cu") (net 8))
 (segment (start 84.517822 120.077822) (end 95.085306 120.077822) (width 0.6) (layer "F.Cu") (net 9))
 (segment (start 95.085306 99.757822) (end 83.496054 99.757822) (width 0.6) (layer "F.Cu") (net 10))
 (segment (start 99.06 68.58) (end 96.8 66.32) (width 0.6) (layer "F.Cu") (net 6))
 (segment (start 99.06 70.485) (end 99.06 68.58) (width 0.6) (layer "F.Cu") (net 6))
 (segment (start 96.8 66.32) (end 96.52 66.32) (width 0.6) (layer "F.Cu") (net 6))
 (segment (start 93.635 75.565) (end 92.68 74.61) (width 0.6) (layer "F.Cu") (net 6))
 (segment (start 97.4725 72.0725) (end 99.06 70.485) (width 0.6) (layer "F.Cu") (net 6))
 (segment (start 99.8725 66.955) (end 100.965 66.955) (width 0.6) (layer "F.Cu") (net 6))
 (segment (start 93.98 75.565) (end 93.635 75.565) (width 0.6) (layer "F.Cu") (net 6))
 (segment (start 99.06 67.7675) (end 99.8725 66.955) (width 0.6) (layer "F.Cu") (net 6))
 (segment (start 99.06 68.58) (end 99.06 67.7675) (width 0.6) (layer "F.Cu") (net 6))
 (via (at 93.98 75.565) (size 0.8) (drill 0.4) (layers "F.Cu" "B.Cu") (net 6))
 (via (at 97.4725 72.0725) (size 0.8) (drill 0.4) (layers "F.Cu" "B.Cu") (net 6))
 (segment (start 97.4725 72.0725) (end 93.98 75.565) (width 0.6) (layer "B.Cu") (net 6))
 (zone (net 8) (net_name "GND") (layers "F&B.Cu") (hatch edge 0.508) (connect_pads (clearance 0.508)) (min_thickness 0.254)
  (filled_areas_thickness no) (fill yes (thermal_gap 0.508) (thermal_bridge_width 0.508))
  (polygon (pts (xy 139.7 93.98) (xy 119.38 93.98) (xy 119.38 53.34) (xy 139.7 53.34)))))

